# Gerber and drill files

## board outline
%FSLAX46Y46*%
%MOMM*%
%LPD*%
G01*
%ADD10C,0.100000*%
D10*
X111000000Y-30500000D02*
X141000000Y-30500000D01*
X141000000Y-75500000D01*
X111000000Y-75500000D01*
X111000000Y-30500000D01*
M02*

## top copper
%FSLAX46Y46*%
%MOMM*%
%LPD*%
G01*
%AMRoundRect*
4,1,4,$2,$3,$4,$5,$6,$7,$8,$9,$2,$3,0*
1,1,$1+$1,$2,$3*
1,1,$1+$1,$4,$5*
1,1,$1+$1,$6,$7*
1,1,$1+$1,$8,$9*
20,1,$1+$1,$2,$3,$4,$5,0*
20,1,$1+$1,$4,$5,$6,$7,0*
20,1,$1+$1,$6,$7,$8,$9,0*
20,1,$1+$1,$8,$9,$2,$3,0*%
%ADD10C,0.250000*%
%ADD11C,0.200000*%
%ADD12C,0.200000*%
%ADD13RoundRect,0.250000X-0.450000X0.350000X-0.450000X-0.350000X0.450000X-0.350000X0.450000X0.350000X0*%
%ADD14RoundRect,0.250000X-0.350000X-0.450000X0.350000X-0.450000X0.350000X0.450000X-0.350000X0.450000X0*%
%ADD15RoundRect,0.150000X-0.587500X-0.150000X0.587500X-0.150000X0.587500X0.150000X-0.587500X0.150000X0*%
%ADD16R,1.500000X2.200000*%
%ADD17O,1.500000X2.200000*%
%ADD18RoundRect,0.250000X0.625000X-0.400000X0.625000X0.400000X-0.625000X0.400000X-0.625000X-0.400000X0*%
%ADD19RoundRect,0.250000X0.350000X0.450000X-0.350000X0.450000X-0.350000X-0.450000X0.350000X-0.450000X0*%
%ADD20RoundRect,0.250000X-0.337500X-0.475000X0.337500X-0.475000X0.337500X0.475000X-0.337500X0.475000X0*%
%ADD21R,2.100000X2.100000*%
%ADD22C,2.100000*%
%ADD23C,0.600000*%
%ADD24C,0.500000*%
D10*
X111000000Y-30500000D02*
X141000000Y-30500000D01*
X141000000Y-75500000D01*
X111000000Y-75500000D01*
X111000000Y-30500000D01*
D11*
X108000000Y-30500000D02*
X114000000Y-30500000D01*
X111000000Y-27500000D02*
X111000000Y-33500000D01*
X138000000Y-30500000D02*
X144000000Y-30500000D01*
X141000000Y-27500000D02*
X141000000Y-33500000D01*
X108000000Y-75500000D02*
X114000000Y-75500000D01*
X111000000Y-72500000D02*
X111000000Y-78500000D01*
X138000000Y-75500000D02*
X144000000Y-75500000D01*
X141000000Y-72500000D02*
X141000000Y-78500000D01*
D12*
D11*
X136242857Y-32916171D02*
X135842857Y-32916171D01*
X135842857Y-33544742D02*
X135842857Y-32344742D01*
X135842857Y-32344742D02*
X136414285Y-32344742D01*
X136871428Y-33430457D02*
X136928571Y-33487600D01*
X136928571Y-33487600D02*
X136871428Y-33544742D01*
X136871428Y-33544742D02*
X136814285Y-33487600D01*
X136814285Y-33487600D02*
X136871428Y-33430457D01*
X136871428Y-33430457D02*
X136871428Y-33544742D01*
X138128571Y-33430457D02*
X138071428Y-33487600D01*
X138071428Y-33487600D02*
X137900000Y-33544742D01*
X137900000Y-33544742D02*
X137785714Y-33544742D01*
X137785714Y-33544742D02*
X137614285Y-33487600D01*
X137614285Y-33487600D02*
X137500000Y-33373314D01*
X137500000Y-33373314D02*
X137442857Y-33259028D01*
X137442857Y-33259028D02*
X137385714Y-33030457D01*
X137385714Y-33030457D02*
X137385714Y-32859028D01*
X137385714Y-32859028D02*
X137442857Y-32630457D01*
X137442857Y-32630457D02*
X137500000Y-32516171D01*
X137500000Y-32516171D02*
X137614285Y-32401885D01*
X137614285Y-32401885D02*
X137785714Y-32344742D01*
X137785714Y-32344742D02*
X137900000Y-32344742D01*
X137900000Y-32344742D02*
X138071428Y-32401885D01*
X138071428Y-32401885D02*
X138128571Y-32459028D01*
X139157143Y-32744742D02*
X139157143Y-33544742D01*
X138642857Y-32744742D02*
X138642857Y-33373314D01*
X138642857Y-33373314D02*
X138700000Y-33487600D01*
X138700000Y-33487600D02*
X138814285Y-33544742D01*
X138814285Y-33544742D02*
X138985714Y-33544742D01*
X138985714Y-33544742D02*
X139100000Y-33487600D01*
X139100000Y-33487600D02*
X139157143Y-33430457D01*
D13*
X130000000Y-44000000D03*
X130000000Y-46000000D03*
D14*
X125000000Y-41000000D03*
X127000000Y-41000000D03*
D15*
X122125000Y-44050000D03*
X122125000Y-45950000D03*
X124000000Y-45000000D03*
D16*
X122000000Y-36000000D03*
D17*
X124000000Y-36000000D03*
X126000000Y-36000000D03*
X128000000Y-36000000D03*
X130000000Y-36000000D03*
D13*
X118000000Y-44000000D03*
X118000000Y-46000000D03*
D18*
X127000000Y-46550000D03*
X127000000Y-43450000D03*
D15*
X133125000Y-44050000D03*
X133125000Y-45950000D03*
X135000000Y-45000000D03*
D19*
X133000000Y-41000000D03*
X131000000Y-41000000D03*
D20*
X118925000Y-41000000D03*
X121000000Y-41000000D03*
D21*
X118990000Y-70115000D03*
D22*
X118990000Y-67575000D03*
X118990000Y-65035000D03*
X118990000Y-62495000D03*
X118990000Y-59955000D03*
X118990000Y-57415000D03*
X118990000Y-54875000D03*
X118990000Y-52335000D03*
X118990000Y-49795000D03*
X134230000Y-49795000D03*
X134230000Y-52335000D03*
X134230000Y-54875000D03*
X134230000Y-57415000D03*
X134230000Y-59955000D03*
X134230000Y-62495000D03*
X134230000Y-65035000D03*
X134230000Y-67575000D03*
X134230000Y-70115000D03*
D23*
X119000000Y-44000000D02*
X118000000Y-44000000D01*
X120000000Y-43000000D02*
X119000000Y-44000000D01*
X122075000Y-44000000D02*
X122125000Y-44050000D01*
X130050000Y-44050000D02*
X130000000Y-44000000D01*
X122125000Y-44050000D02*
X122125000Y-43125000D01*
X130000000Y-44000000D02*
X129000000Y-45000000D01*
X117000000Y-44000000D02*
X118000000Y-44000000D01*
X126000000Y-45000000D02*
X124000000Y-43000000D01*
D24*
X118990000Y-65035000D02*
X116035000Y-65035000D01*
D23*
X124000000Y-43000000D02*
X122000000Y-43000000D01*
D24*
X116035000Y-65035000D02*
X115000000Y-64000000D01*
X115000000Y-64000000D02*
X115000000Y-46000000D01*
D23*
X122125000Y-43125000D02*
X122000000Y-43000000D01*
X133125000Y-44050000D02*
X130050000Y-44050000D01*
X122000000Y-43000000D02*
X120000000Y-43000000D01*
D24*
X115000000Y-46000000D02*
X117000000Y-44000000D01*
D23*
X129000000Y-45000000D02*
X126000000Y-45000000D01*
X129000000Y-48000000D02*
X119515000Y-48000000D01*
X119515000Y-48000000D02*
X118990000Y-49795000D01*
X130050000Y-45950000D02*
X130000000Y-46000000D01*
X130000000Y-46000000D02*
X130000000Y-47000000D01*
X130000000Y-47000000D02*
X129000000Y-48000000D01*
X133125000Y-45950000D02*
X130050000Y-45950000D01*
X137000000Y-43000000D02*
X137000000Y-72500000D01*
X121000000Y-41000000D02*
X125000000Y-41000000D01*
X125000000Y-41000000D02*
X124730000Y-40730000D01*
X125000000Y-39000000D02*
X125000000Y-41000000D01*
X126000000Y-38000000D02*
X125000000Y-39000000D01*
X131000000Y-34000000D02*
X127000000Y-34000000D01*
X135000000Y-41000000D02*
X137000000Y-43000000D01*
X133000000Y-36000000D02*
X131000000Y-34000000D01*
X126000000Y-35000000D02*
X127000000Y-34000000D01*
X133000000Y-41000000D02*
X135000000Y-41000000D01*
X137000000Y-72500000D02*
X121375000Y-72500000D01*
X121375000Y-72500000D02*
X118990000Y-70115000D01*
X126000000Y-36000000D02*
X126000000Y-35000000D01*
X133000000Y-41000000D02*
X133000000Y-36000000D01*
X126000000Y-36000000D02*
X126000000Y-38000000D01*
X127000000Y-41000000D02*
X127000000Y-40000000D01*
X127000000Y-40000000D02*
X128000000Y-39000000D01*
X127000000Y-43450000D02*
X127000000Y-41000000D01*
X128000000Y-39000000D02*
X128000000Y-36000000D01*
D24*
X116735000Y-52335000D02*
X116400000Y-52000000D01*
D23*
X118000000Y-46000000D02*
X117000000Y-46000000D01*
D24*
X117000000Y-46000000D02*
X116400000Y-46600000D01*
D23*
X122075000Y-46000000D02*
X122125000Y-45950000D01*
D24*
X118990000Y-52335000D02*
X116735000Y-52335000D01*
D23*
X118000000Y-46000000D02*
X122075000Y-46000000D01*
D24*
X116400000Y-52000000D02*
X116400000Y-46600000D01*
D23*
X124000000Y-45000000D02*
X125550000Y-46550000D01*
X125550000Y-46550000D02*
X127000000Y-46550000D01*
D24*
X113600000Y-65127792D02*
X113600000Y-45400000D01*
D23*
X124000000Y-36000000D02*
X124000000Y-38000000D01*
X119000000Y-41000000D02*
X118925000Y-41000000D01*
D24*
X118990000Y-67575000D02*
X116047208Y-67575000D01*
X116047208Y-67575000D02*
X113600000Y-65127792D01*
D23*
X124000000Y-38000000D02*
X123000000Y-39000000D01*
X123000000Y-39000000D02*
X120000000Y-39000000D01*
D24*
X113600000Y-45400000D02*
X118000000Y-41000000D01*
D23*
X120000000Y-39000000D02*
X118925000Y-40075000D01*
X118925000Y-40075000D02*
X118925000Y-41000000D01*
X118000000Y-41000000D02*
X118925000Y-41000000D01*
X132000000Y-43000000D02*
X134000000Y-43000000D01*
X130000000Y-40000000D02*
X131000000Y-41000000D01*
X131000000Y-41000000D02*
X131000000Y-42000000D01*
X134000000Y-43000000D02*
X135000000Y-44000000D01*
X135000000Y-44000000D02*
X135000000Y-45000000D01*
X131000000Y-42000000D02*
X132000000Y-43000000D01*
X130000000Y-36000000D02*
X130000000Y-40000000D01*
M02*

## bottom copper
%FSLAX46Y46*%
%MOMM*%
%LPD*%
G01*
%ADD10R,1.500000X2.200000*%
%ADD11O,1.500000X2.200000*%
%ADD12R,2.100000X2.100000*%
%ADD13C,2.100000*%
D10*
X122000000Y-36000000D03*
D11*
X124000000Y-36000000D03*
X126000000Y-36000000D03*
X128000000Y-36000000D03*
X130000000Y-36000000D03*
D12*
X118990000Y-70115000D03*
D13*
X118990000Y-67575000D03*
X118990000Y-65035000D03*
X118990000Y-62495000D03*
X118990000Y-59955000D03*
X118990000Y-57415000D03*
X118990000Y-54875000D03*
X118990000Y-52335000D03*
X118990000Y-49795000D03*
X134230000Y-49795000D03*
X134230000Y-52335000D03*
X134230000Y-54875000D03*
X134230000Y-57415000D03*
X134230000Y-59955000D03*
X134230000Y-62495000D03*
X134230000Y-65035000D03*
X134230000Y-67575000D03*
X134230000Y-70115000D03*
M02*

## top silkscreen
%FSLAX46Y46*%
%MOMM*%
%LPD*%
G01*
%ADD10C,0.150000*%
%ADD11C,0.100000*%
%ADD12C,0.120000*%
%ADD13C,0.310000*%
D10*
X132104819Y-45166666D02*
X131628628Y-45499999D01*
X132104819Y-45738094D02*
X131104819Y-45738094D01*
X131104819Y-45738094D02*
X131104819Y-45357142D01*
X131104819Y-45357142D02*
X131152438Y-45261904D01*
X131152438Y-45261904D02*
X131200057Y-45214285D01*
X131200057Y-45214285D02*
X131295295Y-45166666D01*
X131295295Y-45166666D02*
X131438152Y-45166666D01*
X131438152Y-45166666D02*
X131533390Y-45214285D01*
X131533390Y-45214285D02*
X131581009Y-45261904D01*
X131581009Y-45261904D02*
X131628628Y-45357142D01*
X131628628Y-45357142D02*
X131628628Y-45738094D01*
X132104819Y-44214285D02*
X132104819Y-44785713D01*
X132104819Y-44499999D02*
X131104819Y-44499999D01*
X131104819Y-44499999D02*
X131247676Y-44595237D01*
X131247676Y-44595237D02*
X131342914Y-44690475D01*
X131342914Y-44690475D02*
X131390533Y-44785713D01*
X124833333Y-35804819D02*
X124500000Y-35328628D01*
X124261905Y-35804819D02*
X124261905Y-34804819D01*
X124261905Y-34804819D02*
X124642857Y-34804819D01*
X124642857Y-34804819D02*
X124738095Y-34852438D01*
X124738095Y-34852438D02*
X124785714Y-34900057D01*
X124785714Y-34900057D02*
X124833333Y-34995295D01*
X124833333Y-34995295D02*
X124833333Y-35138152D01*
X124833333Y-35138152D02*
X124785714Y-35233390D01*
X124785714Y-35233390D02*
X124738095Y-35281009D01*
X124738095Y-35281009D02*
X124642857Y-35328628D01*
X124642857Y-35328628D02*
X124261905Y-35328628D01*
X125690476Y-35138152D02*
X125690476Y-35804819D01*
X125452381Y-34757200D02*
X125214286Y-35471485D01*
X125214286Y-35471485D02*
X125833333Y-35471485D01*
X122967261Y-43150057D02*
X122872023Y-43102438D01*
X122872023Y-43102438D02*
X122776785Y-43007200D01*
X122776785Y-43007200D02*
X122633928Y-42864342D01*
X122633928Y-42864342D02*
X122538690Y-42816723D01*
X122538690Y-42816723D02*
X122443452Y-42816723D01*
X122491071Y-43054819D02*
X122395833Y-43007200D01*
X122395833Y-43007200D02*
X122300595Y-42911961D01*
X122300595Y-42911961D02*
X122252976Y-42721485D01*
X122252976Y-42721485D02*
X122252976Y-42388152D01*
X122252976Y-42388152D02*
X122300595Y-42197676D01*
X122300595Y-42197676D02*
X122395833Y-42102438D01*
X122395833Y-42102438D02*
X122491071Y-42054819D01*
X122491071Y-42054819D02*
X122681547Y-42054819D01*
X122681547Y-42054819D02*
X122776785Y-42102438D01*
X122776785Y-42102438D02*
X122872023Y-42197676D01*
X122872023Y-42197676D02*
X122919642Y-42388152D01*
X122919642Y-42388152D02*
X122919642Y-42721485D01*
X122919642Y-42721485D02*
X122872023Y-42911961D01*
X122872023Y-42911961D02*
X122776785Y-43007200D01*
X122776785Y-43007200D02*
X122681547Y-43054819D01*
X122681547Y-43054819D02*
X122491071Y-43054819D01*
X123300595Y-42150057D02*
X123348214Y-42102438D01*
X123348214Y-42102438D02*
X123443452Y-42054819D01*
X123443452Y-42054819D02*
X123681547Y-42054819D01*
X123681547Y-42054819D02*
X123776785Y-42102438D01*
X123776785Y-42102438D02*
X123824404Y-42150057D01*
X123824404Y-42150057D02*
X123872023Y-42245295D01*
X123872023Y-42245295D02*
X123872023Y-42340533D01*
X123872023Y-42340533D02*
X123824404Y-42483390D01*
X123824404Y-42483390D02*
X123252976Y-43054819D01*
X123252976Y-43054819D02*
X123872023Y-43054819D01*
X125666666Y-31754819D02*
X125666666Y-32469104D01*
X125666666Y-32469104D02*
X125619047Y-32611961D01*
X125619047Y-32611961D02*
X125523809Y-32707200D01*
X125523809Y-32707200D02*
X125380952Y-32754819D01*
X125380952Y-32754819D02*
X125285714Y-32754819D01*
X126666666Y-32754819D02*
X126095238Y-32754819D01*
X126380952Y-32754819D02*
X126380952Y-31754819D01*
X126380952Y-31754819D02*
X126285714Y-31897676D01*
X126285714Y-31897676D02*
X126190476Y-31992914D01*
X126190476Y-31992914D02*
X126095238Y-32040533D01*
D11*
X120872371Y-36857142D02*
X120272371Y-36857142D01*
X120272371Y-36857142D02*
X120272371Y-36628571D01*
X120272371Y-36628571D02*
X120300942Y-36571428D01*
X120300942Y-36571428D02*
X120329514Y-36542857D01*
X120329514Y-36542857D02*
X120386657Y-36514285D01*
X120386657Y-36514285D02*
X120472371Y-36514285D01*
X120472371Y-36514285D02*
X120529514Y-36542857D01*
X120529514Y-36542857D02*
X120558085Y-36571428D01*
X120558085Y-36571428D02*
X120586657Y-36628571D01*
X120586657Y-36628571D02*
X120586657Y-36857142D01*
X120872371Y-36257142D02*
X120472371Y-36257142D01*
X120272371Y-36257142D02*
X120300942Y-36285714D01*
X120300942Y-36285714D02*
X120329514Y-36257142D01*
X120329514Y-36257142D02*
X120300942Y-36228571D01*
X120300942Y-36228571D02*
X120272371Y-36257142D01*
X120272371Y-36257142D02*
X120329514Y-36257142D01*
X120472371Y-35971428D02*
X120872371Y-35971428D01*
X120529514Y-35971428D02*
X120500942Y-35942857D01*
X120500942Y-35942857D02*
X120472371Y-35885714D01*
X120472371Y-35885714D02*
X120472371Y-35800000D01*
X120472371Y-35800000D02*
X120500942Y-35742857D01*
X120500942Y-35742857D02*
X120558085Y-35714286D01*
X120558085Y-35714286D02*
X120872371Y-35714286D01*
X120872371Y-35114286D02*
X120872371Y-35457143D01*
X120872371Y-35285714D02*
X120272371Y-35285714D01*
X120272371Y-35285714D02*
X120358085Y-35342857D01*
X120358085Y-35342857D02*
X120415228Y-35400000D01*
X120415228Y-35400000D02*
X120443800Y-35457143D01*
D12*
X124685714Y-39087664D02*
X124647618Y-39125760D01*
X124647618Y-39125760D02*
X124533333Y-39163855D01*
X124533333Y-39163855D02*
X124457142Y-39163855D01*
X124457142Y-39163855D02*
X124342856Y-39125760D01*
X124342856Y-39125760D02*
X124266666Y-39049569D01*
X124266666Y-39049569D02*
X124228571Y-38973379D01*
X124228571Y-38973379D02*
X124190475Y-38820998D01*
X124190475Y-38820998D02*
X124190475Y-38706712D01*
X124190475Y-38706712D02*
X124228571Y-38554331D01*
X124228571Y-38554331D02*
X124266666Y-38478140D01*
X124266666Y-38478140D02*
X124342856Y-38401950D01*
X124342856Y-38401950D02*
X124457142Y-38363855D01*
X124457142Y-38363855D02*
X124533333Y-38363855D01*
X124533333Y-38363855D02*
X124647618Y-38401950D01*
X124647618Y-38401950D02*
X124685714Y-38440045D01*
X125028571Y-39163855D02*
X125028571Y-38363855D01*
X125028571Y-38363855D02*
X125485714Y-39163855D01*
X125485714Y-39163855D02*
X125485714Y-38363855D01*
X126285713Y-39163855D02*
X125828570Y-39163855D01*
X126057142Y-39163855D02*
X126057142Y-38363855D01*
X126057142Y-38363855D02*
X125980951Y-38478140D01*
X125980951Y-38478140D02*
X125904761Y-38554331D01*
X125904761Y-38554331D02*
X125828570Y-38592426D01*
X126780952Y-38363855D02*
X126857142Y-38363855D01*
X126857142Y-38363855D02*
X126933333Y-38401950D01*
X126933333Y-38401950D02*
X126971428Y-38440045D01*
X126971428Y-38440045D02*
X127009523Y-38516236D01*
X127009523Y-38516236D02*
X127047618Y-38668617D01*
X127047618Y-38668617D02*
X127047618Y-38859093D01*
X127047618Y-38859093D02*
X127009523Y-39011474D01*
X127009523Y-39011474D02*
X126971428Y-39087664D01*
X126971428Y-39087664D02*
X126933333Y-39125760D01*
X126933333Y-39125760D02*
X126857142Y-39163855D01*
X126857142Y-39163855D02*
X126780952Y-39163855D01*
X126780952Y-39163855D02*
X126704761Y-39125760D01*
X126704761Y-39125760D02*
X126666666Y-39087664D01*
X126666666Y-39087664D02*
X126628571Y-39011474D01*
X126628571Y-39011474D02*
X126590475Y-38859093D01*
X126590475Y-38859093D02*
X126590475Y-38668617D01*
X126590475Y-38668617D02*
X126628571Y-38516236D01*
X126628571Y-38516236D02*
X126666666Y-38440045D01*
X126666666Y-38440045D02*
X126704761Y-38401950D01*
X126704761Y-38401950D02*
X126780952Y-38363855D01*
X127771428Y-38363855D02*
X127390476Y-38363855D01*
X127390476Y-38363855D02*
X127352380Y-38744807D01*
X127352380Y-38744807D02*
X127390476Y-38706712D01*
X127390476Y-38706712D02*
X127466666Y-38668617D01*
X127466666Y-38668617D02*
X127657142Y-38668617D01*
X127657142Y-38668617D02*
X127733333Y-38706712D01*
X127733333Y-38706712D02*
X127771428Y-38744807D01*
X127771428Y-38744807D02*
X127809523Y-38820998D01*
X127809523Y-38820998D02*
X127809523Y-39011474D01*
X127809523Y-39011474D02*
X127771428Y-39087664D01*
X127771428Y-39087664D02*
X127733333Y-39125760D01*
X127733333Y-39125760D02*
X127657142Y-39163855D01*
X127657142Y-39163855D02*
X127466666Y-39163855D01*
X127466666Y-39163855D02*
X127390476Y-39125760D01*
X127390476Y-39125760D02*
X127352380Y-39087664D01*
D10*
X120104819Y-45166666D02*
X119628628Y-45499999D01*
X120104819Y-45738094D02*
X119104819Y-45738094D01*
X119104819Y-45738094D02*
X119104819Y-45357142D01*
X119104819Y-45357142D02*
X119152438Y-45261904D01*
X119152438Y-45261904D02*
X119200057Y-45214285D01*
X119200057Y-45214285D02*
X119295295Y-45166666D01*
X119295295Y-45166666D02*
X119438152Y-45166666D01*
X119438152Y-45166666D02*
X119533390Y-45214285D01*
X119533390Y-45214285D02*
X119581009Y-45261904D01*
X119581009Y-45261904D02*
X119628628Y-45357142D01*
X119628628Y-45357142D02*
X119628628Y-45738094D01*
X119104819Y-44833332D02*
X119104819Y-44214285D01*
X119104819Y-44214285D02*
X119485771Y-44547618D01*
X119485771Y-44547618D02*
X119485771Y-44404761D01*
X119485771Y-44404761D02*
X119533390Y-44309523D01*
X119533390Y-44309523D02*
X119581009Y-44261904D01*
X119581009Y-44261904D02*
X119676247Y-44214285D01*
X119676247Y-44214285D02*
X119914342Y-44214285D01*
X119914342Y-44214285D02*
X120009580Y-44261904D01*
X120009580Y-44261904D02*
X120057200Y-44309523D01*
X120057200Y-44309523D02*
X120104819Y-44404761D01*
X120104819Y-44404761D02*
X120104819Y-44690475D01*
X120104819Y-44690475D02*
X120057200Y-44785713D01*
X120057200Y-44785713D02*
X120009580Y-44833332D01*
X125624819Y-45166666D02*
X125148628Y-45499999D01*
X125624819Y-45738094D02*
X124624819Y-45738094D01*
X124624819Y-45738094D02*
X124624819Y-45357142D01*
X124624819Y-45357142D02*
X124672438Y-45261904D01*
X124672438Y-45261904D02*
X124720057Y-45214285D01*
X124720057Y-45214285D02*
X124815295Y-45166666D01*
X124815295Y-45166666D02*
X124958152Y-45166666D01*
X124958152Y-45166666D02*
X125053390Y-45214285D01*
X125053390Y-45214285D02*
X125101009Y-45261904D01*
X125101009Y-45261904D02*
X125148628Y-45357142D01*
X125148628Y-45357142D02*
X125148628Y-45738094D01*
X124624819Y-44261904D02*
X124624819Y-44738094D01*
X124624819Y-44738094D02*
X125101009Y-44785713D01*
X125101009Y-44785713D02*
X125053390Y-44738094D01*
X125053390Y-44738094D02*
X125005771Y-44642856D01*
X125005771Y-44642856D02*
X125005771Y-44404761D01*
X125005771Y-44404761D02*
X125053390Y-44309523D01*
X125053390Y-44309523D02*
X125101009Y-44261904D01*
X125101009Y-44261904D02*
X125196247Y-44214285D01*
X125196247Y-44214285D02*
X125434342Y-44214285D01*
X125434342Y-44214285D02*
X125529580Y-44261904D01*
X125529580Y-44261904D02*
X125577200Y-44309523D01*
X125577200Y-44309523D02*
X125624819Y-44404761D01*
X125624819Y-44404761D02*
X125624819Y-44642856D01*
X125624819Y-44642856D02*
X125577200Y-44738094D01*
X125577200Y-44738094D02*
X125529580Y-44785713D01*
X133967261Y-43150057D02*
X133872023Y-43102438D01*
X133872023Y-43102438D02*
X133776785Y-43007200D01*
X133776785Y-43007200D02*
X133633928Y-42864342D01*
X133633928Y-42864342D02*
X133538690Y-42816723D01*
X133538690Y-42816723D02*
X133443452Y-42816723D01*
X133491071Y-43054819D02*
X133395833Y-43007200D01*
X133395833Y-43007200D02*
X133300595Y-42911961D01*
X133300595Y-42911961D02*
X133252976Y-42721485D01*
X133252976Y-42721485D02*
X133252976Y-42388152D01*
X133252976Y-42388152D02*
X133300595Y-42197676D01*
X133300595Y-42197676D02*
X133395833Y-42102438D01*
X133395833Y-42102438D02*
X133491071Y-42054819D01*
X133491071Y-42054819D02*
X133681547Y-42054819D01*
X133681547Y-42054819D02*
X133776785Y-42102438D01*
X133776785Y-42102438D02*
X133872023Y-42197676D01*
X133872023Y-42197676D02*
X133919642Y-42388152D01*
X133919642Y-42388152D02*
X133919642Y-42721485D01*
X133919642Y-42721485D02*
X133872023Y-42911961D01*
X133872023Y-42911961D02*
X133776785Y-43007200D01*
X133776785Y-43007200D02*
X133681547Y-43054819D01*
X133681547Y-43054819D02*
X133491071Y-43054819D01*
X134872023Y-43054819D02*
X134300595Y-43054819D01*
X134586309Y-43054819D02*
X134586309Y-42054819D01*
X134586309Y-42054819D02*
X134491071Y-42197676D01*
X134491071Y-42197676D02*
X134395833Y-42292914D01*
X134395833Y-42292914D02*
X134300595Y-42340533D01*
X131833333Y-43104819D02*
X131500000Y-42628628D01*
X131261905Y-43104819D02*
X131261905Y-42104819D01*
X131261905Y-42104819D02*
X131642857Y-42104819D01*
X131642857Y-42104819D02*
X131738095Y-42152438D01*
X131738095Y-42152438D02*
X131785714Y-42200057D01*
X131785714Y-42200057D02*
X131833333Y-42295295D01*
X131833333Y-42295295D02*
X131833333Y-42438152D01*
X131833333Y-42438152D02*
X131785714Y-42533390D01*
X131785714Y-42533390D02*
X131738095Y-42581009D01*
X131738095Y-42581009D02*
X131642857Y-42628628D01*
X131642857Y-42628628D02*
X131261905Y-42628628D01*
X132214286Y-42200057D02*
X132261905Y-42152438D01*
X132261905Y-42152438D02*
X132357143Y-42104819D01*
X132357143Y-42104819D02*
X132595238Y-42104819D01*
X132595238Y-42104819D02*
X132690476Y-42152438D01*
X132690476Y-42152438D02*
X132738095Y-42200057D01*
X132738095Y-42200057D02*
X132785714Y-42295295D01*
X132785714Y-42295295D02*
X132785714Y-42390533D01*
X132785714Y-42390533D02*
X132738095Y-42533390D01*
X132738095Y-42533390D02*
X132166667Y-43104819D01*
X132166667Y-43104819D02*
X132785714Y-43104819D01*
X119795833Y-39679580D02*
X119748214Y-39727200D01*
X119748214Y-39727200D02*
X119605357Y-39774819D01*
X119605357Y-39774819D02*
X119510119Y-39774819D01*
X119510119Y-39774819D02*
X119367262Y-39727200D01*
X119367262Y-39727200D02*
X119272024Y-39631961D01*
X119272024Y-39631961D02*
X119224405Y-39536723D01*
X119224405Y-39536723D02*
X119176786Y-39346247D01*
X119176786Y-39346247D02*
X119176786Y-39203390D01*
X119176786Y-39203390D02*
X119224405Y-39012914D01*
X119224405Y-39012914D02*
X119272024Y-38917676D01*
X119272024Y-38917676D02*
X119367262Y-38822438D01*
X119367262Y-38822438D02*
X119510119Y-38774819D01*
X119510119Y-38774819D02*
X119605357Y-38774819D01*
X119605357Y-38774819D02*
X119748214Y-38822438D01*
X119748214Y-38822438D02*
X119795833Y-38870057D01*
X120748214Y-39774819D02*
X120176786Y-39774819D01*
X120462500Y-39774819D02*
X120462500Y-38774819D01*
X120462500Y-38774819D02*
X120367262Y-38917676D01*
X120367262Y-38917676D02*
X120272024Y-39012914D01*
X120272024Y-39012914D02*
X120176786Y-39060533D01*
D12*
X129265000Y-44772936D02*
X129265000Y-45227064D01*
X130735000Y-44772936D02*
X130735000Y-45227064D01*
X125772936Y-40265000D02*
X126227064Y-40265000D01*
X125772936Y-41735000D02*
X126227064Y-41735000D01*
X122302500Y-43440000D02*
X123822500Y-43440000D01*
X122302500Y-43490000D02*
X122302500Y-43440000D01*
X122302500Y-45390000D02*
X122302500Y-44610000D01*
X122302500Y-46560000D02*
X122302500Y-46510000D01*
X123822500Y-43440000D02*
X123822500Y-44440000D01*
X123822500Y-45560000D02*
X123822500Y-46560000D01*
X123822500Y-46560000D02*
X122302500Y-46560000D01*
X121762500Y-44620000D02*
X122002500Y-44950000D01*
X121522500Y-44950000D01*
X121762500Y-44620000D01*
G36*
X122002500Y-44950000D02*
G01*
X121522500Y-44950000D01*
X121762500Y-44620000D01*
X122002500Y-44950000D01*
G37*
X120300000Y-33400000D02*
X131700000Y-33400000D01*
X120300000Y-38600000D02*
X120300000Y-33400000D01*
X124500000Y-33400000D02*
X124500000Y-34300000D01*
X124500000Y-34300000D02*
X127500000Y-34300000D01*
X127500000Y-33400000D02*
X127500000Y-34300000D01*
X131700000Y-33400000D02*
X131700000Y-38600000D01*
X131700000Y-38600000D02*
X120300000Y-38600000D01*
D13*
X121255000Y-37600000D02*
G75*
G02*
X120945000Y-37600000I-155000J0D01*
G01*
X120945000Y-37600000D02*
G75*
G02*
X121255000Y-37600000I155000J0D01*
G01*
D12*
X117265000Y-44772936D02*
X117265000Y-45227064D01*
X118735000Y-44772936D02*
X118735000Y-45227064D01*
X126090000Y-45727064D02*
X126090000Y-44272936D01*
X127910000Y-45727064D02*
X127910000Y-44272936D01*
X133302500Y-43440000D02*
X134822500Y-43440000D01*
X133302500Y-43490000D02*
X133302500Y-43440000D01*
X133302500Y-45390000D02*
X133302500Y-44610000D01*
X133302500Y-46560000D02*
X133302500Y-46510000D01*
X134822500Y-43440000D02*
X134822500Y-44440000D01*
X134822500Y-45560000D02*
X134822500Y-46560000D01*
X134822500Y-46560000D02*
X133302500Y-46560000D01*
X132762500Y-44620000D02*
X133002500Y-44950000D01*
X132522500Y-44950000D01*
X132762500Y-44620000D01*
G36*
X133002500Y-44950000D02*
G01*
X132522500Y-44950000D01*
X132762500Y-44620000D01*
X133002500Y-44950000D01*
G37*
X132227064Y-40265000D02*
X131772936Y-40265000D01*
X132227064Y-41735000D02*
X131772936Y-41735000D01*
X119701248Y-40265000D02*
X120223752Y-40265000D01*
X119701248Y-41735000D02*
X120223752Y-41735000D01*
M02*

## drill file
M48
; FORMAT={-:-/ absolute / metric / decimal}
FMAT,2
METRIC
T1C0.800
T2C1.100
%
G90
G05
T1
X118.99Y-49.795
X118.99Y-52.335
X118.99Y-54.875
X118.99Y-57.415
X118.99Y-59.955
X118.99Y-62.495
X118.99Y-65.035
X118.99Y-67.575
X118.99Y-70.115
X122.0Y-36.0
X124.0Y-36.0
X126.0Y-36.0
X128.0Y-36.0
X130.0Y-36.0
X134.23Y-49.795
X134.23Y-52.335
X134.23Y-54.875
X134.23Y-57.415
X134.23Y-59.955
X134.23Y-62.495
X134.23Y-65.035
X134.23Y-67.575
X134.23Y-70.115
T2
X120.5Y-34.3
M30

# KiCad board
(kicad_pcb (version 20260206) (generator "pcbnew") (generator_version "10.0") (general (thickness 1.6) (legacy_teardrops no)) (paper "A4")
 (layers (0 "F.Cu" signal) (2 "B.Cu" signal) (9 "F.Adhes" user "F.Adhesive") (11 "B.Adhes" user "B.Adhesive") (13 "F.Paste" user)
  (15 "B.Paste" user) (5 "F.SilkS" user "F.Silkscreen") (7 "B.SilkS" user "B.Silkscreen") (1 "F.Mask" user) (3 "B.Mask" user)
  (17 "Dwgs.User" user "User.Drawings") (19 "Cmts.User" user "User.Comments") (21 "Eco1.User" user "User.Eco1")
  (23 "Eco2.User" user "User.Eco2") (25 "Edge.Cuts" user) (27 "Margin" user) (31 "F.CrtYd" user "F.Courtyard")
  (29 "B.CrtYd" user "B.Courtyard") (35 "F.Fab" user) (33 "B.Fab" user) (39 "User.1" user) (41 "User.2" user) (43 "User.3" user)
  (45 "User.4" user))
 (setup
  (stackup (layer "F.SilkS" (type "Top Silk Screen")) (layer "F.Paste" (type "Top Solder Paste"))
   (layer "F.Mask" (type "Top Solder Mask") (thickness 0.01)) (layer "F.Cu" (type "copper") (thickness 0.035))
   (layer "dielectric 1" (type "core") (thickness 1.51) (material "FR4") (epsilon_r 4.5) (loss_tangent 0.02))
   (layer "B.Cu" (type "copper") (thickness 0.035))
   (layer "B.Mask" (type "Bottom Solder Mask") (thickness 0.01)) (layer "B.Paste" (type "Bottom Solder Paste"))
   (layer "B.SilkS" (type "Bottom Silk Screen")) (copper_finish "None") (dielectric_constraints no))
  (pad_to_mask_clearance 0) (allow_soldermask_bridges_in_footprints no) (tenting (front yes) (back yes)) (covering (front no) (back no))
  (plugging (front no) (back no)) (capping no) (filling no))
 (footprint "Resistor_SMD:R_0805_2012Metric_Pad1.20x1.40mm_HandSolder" (layer "F.Cu") (at 130 45 -90)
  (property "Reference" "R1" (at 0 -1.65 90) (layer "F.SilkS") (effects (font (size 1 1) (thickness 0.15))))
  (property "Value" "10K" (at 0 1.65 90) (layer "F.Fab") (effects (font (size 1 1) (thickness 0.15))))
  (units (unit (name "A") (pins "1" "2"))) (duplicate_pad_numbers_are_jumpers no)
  (fp_line (start -0.227064 0.735) (end 0.227064 0.735) (stroke (width 0.12) (type solid)) (layer "F.SilkS"))
  (fp_line (start -0.227064 -0.735) (end 0.227064 -0.735) (stroke (width 0.12) (type solid)) (layer "F.SilkS"))
  (pad "1" smd roundrect (at -1 0 270) (size 1.2 1.4) (layers "F.Cu" "F.Mask" "F.Paste") (roundrect_rratio 0.208333) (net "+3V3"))
  (pad "2" smd roundrect (at 1 0 270) (size 1.2 1.4) (layers "F.Cu" "F.Mask" "F.Paste") (roundrect_rratio 0.208333) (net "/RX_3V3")))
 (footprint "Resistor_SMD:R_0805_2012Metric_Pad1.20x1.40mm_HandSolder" (layer "F.Cu") (at 126 41)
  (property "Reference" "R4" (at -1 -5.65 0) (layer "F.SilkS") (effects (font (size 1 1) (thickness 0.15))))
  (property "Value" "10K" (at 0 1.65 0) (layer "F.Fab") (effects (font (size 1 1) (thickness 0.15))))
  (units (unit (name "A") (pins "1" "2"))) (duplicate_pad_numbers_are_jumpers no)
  (fp_line (start -0.227064 -0.735) (end 0.227064 -0.735) (stroke (width 0.12) (type solid)) (layer "F.SilkS"))
  (fp_line (start -0.227064 0.735) (end 0.227064 0.735) (stroke (width 0.12) (type solid)) (layer "F.SilkS"))
  (pad "1" smd roundrect (at -1 0) (size 1.2 1.4) (layers "F.Cu" "F.Mask" "F.Paste") (roundrect_rratio 0.208333) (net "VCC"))
  (pad "2" smd roundrect (at 1 0) (size 1.2 1.4) (layers "F.Cu" "F.Mask" "F.Paste") (roundrect_rratio 0.208333) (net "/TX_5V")))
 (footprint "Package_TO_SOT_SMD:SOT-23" (layer "F.Cu") (at 123.0625 45)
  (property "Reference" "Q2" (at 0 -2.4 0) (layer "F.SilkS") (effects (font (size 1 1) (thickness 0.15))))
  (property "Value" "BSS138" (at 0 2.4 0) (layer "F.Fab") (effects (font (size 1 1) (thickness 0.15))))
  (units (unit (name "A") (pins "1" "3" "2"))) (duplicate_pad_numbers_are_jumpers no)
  (fp_line (start -0.76 -1.56) (end 0.76 -1.56) (stroke (width 0.12) (type solid)) (layer "F.SilkS"))
  (fp_line (start -0.76 -1.51) (end -0.76 -1.56) (stroke (width 0.12) (type solid)) (layer "F.SilkS"))
  (fp_line (start -0.76 0.39) (end -0.76 -0.39) (stroke (width 0.12) (type solid)) (layer "F.SilkS"))
  (fp_line (start -0.76 1.56) (end -0.76 1.51) (stroke (width 0.12) (type solid)) (layer "F.SilkS"))
  (fp_line (start 0.76 -1.56) (end 0.76 -0.56) (stroke (width 0.12) (type solid)) (layer "F.SilkS"))
  (fp_line (start 0.76 0.56) (end 0.76 1.56) (stroke (width 0.12) (type solid)) (layer "F.SilkS"))
  (fp_line (start 0.76 1.56) (end -0.76 1.56) (stroke (width 0.12) (type solid)) (layer "F.SilkS"))
  (fp_poly (pts (xy -1.3 -0.38) (xy -1.06 -0.05) (xy -1.54 -0.05)) (stroke (width 0.12) (type solid)) (fill yes) (layer "F.SilkS"))
  (pad "1" smd roundrect (at -0.9375 -0.95) (size 1.475 0.6) (layers "F.Cu" "F.Mask" "F.Paste") (roundrect_rratio 0.25) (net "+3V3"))
  (pad "2" smd roundrect (at -0.9375 0.95) (size 1.475 0.6) (layers "F.Cu" "F.Mask" "F.Paste") (roundrect_rratio 0.25) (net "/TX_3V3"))
  (pad "3" smd roundrect (at 0.9375 0) (size 1.475 0.6) (layers "F.Cu" "F.Mask" "F.Paste") (roundrect_rratio 0.25) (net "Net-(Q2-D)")))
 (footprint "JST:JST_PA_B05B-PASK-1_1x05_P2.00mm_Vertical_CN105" (layer "F.Cu") (at 122 36)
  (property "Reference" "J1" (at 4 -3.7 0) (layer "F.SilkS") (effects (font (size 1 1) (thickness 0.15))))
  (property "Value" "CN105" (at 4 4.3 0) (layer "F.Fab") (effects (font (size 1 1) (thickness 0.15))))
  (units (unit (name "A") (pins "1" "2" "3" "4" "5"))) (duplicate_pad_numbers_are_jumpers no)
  (fp_line (start -1.7 -2.6) (end 9.7 -2.6) (stroke (width 0.12) (type solid)) (layer "F.SilkS"))
  (fp_line (start -1.7 2.6) (end -1.7 -2.6) (stroke (width 0.12) (type solid)) (layer "F.SilkS"))
  (fp_line (start 2.5 -2.6) (end 2.5 -1.7) (stroke (width 0.12) (type solid)) (layer "F.SilkS"))
  (fp_line (start 2.5 -1.7) (end 5.5 -1.7) (stroke (width 0.12) (type solid)) (layer "F.SilkS"))
  (fp_line (start 5.5 -2.6) (end 5.5 -1.7) (stroke (width 0.12) (type solid)) (layer "F.SilkS"))
  (fp_line (start 9.7 -2.6) (end 9.7 2.6) (stroke (width 0.12) (type solid)) (layer "F.SilkS"))
  (fp_line (start 9.7 2.6) (end -1.7 2.6) (stroke (width 0.12) (type solid)) (layer "F.SilkS"))
  (fp_circle (center -0.9 1.6) (end -0.65 1.6) (stroke (width 0.12) (type solid)) (fill yes) (layer "F.SilkS"))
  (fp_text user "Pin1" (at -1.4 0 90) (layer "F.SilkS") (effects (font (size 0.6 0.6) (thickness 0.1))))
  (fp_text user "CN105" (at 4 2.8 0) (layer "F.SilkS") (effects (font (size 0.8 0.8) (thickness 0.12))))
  (pad "" np_thru_hole circle (at -1.5 -1.7) (size 1.1 1.1) (drill 1.1) (layers "*.Cu" "*.Mask"))
  (pad "1" thru_hole rect (at 0 0) (size 1.5 2.2) (drill 0.8) (layers "*.Cu" "*.Mask") (remove_unused_layers no)
   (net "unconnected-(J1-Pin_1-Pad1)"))
  (pad "2" thru_hole oval (at 2 0) (size 1.5 2.2) (drill 0.8) (layers "*.Cu" "*.Mask") (remove_unused_layers no) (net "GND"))
  (pad "3" thru_hole oval (at 4 0) (size 1.5 2.2) (drill 0.8) (layers "*.Cu" "*.Mask") (remove_unused_layers no) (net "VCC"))
  (pad "4" thru_hole oval (at 6 0) (size 1.5 2.2) (drill 0.8) (layers "*.Cu" "*.Mask") (remove_unused_layers no) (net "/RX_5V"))
  (pad "5" thru_hole oval (at 8 0) (size 1.5 2.2) (drill 0.8) (layers "*.Cu" "*.Mask") (remove_unused_layers no) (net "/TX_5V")))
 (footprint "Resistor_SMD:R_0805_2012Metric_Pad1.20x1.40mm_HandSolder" (layer "F.Cu") (at 118 45 -90)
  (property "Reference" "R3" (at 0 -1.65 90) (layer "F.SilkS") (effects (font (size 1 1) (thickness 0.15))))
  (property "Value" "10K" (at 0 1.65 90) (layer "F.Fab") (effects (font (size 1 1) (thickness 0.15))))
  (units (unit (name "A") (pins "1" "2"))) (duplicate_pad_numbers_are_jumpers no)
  (fp_line (start -0.227064 0.735) (end 0.227064 0.735) (stroke (width 0.12) (type solid)) (layer "F.SilkS"))
  (fp_line (start -0.227064 -0.735) (end 0.227064 -0.735) (stroke (width 0.12) (type solid)) (layer "F.SilkS"))
  (pad "1" smd roundrect (at -1 0 270) (size 1.2 1.4) (layers "F.Cu" "F.Mask" "F.Paste") (roundrect_rratio 0.208333) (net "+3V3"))
  (pad "2" smd roundrect (at 1 0 270) (size 1.2 1.4) (layers "F.Cu" "F.Mask" "F.Paste") (roundrect_rratio 0.208333) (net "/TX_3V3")))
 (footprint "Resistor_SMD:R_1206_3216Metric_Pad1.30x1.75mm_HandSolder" (layer "F.Cu") (at 127 45 90)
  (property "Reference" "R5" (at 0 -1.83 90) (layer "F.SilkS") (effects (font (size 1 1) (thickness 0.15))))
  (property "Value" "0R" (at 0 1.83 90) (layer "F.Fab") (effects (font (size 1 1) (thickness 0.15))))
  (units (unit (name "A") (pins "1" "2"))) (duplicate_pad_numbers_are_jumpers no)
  (fp_line (start -0.727064 -0.91) (end 0.727064 -0.91) (stroke (width 0.12) (type solid)) (layer "F.SilkS"))
  (fp_line (start -0.727064 0.91) (end 0.727064 0.91) (stroke (width 0.12) (type solid)) (layer "F.SilkS"))
  (pad "1" smd roundrect (at -1.55 0 90) (size 1.3 1.75) (layers "F.Cu" "F.Mask" "F.Paste") (roundrect_rratio 0.192308) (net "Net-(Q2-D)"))
  (pad "2" smd roundrect (at 1.55 0 90) (size 1.3 1.75) (layers "F.Cu" "F.Mask" "F.Paste") (roundrect_rratio 0.192308) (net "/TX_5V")))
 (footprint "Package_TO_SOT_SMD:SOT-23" (layer "F.Cu") (at 134.0625 45)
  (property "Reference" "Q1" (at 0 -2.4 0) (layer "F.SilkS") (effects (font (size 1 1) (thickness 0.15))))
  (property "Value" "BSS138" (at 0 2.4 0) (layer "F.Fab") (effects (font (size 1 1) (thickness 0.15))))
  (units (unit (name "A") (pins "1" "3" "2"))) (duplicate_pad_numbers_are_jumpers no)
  (fp_line (start -0.76 -1.56) (end 0.76 -1.56) (stroke (width 0.12) (type solid)) (layer "F.SilkS"))
  (fp_line (start -0.76 -1.51) (end -0.76 -1.56) (stroke (width 0.12) (type solid)) (layer "F.SilkS"))
  (fp_line (start -0.76 0.39) (end -0.76 -0.39) (stroke (width 0.12) (type solid)) (layer "F.SilkS"))
  (fp_line (start -0.76 1.56) (end -0.76 1.51) (stroke (width 0.12) (type solid)) (layer "F.SilkS"))
  (fp_line (start 0.76 -1.56) (end 0.76 -0.56) (stroke (width 0.12) (type solid)) (layer "F.SilkS"))
  (fp_line (start 0.76 0.56) (end 0.76 1.56) (stroke (width 0.12) (type solid)) (layer "F.SilkS"))
  (fp_line (start 0.76 1.56) (end -0.76 1.56) (stroke (width 0.12) (type solid)) (layer "F.SilkS"))
  (fp_poly (pts (xy -1.3 -0.38) (xy -1.06 -0.05) (xy -1.54 -0.05)) (stroke (width 0.12) (type solid)) (fill yes) (layer "F.SilkS"))
  (pad "1" smd roundrect (at -0.9375 -0.95) (size 1.475 0.6) (layers "F.Cu" "F.Mask" "F.Paste") (roundrect_rratio 0.25) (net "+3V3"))
  (pad "2" smd roundrect (at -0.9375 0.95) (size 1.475 0.6) (layers "F.Cu" "F.Mask" "F.Paste") (roundrect_rratio 0.25) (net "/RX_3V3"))
  (pad "3" smd roundrect (at 0.9375 0) (size 1.475 0.6) (layers "F.Cu" "F.Mask" "F.Paste") (roundrect_rratio 0.25) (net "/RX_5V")))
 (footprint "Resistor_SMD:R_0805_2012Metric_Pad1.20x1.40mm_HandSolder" (layer "F.Cu") (at 132 41 180)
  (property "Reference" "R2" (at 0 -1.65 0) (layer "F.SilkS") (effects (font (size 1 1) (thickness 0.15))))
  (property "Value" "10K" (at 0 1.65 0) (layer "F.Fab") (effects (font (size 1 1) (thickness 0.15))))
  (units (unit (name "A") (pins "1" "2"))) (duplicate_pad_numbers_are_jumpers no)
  (fp_line (start -0.227064 0.735) (end 0.227064 0.735) (stroke (width 0.12) (type solid)) (layer "F.SilkS"))
  (fp_line (start -0.227064 -0.735) (end 0.227064 -0.735) (stroke (width 0.12) (type solid)) (layer "F.SilkS"))
  (pad "1" smd roundrect (at -1 0 180) (size 1.2 1.4) (layers "F.Cu" "F.Mask" "F.Paste") (roundrect_rratio 0.208333) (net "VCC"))
  (pad "2" smd roundrect (at 1 0 180) (size 1.2 1.4) (layers "F.Cu" "F.Mask" "F.Paste") (roundrect_rratio 0.208333) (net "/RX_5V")))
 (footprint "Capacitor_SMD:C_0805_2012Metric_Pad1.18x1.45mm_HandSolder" (layer "F.Cu") (at 119.9625 41)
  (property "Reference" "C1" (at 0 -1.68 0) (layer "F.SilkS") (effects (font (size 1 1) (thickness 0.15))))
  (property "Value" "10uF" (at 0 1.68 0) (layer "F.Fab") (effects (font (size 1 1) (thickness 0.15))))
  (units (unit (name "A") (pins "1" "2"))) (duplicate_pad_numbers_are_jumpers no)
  (fp_line (start -0.261252 -0.735) (end 0.261252 -0.735) (stroke (width 0.12) (type solid)) (layer "F.SilkS"))
  (fp_line (start -0.261252 0.735) (end 0.261252 0.735) (stroke (width 0.12) (type solid)) (layer "F.SilkS"))
  (pad "1" smd roundrect (at -1.0375 0) (size 1.175 1.45) (layers "F.Cu" "F.Mask" "F.Paste") (roundrect_rratio 0.212766) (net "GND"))
  (pad "2" smd roundrect (at 1.0375 0) (size 1.175 1.45) (layers "F.Cu" "F.Mask" "F.Paste") (roundrect_rratio 0.212766) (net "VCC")))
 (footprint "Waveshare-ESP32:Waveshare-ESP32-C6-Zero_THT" (layer "B.Cu") (at 126.61 70.115)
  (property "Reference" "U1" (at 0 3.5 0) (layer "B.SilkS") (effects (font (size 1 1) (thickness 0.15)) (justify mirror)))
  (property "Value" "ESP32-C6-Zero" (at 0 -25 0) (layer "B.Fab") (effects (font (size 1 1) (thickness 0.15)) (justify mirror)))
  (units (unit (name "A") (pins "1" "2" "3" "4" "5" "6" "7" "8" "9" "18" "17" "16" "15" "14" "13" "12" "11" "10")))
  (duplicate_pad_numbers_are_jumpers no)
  (pad "1" thru_hole rect (at -7.62 0) (size 2.1 2.1) (drill 0.8) (layers "*.Cu" "*.Mask") (remove_unused_layers no) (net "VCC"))
  (pad "2" thru_hole circle (at -7.62 -2.54) (size 2.1 2.1) (drill 0.8) (layers "*.Cu" "*.Mask") (remove_unused_layers no) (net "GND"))
  (pad "3" thru_hole circle (at -7.62 -5.08) (size 2.1 2.1) (drill 0.8) (layers "*.Cu" "*.Mask") (remove_unused_layers no) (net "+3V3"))
  (pad "4" thru_hole circle (at -7.62 -7.62) (size 2.1 2.1) (drill 0.8) (layers "*.Cu" "*.Mask") (remove_unused_layers no)
   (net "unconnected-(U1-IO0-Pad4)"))
  (pad "5" thru_hole circle (at -7.62 -10.16) (size 2.1 2.1) (drill 0.8) (layers "*.Cu" "*.Mask") (remove_unused_layers no)
   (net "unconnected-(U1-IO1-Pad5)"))
  (pad "6" thru_hole circle (at -7.62 -12.7) (size 2.1 2.1) (drill 0.8) (layers "*.Cu" "*.Mask") (remove_unused_layers no)
   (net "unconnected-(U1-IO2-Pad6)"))
  (pad "7" thru_hole circle (at -7.62 -15.24) (size 2.1 2.1) (drill 0.8) (layers "*.Cu" "*.Mask") (remove_unused_layers no)
   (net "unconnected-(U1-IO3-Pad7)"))
  (pad "8" thru_hole circle (at -7.62 -17.78) (size 2.1 2.1) (drill 0.8) (layers "*.Cu" "*.Mask") (remove_unused_layers no) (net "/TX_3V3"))
  (pad "9" thru_hole circle (at -7.62 -20.32) (size 2.1 2.1) (drill 0.8) (layers "*.Cu" "*.Mask") (remove_unused_layers no) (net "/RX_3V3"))
  (pad "10" thru_hole circle (at 7.62 -20.32) (size 2.1 2.1) (drill 0.8) (layers "*.Cu" "*.Mask") (remove_unused_layers no)
   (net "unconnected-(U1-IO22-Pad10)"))
  (pad "11" thru_hole circle (at 7.62 -17.78) (size 2.1 2.1) (drill 0.8) (layers "*.Cu" "*.Mask") (remove_unused_layers no)
   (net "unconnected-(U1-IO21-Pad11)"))
  (pad "12" thru_hole circle (at 7.62 -15.24) (size 2.1 2.1) (drill 0.8) (layers "*.Cu" "*.Mask") (remove_unused_layers no)
   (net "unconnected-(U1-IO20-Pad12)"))
  (pad "13" thru_hole circle (at 7.62 -12.7) (size 2.1 2.1) (drill 0.8) (layers "*.Cu" "*.Mask") (remove_unused_layers no)
   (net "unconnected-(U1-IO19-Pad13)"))
  (pad "14" thru_hole circle (at 7.62 -10.16) (size 2.1 2.1) (drill 0.8) (layers "*.Cu" "*.Mask") (remove_unused_layers no)
   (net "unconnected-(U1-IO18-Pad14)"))
  (pad "15" thru_hole circle (at 7.62 -7.62) (size 2.1 2.1) (drill 0.8) (layers "*.Cu" "*.Mask") (remove_unused_layers no)
   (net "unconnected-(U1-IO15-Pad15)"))
  (pad "16" thru_hole circle (at 7.62 -5.08) (size 2.1 2.1) (drill 0.8) (layers "*.Cu" "*.Mask") (remove_unused_layers no)
   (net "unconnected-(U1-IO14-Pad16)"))
  (pad "17" thru_hole circle (at 7.62 -2.54) (size 2.1 2.1) (drill 0.8) (layers "*.Cu" "*.Mask") (remove_unused_layers no)
   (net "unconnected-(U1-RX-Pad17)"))
  (pad "18" thru_hole circle (at 7.62 0) (size 2.1 2.1) (drill 0.8) (layers "*.Cu" "*.Mask") (remove_unused_layers no)
   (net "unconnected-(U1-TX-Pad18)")))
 (gr_rect (start 111 30.5) (end 141 75.5) (stroke (width 0.1) (type default)) (fill no) (layer "Edge.Cuts"))
 (gr_rect (start 111 30.5) (end 141 75.5) (stroke (width 0.25) (type default)) (fill no) (layer "F.Cu"))
 (gr_line (start 108 30.5) (end 114 30.5) (stroke (width 0.2) (type default)) (layer "F.Cu"))
 (gr_line (start 111 27.5) (end 111 33.5) (stroke (width 0.2) (type default)) (layer "F.Cu"))
 (gr_line (start 138 30.5) (end 144 30.5) (stroke (width 0.2) (type default)) (layer "F.Cu"))
 (gr_line (start 141 27.5) (end 141 33.5) (stroke (width 0.2) (type default)) (layer "F.Cu"))
 (gr_line (start 108 75.5) (end 114 75.5) (stroke (width 0.2) (type default)) (layer "F.Cu"))
 (gr_line (start 111 72.5) (end 111 78.5) (stroke (width 0.2) (type default)) (layer "F.Cu"))
 (gr_line (start 138 75.5) (end 144 75.5) (stroke (width 0.2) (type default)) (layer "F.Cu"))
 (gr_line (start 141 72.5) (end 141 78.5) (stroke (width 0.2) (type default)) (layer "F.Cu"))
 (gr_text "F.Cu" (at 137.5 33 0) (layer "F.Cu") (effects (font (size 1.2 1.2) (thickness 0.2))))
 (segment (start 119 44) (end 118 44) (width 0.6) (layer "F.Cu") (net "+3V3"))
 (segment (start 120 43) (end 119 44) (width 0.6) (layer "F.Cu") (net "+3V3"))
 (segment (start 122.075 44) (end 122.125 44.05) (width 0.6) (layer "F.Cu") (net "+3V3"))
 (segment (start 130.05 44.05) (end 130 44) (width 0.6) (layer "F.Cu") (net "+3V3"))
 (segment (start 122.125 44.05) (end 122.125 43.125) (width 0.6) (layer "F.Cu") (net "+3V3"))
 (segment (start 130 44) (end 129 45) (width 0.6) (layer "F.Cu") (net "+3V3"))
 (segment (start 117 44) (end 118 44) (width 0.6) (layer "F.Cu") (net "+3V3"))
 (segment (start 126 45) (end 124 43) (width 0.6) (layer "F.Cu") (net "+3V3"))
 (segment (start 118.99 65.035) (end 116.035 65.035) (width 0.5) (layer "F.Cu") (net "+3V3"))
 (segment (start 124 43) (end 122 43) (width 0.6) (layer "F.Cu") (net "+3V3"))
 (segment (start 116.035 65.035) (end 115 64) (width 0.5) (layer "F.Cu") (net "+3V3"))
 (segment (start 115 64) (end 115 46) (width 0.5) (layer "F.Cu") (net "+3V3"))
 (segment (start 122.125 43.125) (end 122 43) (width 0.6) (layer "F.Cu") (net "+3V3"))
 (segment (start 133.125 44.05) (end 130.05 44.05) (width 0.6) (layer "F.Cu") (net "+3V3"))
 (segment (start 122 43) (end 120 43) (width 0.6) (layer "F.Cu") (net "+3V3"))
 (segment (start 115 46) (end 117 44) (width 0.5) (layer "F.Cu") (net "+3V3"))
 (segment (start 129 45) (end 126 45) (width 0.6) (layer "F.Cu") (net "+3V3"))
 (segment (start 129 48) (end 119.515 48) (width 0.6) (layer "F.Cu") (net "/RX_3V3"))
 (segment (start 119.515 48) (end 118.99 49.795) (width 0.6) (layer "F.Cu") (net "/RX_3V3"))
 (segment (start 130.05 45.95) (end 130 46) (width 0.6) (layer "F.Cu") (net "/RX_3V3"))
 (segment (start 130 46) (end 130 47) (width 0.6) (layer "F.Cu") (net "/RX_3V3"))
 (segment (start 130 47) (end 129 48) (width 0.6) (layer "F.Cu") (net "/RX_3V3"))
 (segment (start 133.125 45.95) (end 130.05 45.95) (width 0.6) (layer "F.Cu") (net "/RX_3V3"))
 (segment (start 137 43) (end 137 72.5) (width 0.6) (layer "F.Cu") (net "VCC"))
 (segment (start 121 41) (end 125 41) (width 0.6) (layer "F.Cu") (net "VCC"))
 (segment (start 125 41) (end 124.73 40.73) (width 0.6) (layer "F.Cu") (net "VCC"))
 (segment (start 125 39) (end 125 41) (width 0.6) (layer "F.Cu") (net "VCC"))
 (segment (start 126 38) (end 125 39) (width 0.6) (layer "F.Cu") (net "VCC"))
 (segment (start 131 34) (end 127 34) (width 0.6) (layer "F.Cu") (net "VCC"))
 (segment (start 135 41) (end 137 43) (width 0.6) (layer "F.Cu") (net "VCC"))
 (segment (start 133 36) (end 131 34) (width 0.6) (layer "F.Cu") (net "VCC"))
 (segment (start 126 35) (end 127 34) (width 0.6) (layer "F.Cu") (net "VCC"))
 (segment (start 133 41) (end 135 41) (width 0.6) (layer "F.Cu") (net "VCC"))
 (segment (start 137 72.5) (end 121.375 72.5) (width 0.6) (layer "F.Cu") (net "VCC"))
 (segment (start 121.375 72.5) (end 118.99 70.115) (width 0.6) (layer "F.Cu") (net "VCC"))
 (segment (start 126 36) (end 126 35) (width 0.6) (layer "F.Cu") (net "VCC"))
 (segment (start 133 41) (end 133 36) (width 0.6) (layer "F.Cu") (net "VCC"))
 (segment (start 126 36) (end 126 38) (width 0.6) (layer "F.Cu") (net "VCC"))
 (segment (start 127 41) (end 127 40) (width 0.6) (layer "F.Cu") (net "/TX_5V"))
 (segment (start 127 40) (end 128 39) (width 0.6) (layer "F.Cu") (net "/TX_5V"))
 (segment (start 127 43.45) (end 127 41) (width 0.6) (layer "F.Cu") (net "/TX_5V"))
 (segment (start 128 39) (end 128 36) (width 0.6) (layer "F.Cu") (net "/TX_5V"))
 (segment (start 116.735 52.335) (end 116.4 52) (width 0.5) (layer "F.Cu") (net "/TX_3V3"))
 (segment (start 118 46) (end 117 46) (width 0.6) (layer "F.Cu") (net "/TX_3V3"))
 (segment (start 117 46) (end 116.4 46.6) (width 0.5) (layer "F.Cu") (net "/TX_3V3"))
 (segment (start 122.075 46) (end 122.125 45.95) (width 0.6) (layer "F.Cu") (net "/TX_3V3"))
 (segment (start 118.99 52.335) (end 116.735 52.335) (width 0.5) (layer "F.Cu") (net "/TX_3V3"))
 (segment (start 118 46) (end 122.075 46) (width 0.6) (layer "F.Cu") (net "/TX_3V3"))
 (segment (start 116.4 52) (end 116.4 46.6) (width 0.5) (layer "F.Cu") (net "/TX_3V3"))
 (segment (start 124 45) (end 125.55 46.55) (width 0.6) (layer "F.Cu") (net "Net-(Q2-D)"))
 (segment (start 125.55 46.55) (end 127 46.55) (width 0.6) (layer "F.Cu") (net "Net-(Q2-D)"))
 (segment (start 113.6 65.127792) (end 113.6 45.4) (width 0.5) (layer "F.Cu") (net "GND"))
 (segment (start 124 36) (end 124 38) (width 0.6) (layer "F.Cu") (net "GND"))
 (segment (start 119 41) (end 118.925 41) (width 0.6) (layer "F.Cu") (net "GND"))
 (segment (start 118.99 67.575) (end 116.047208 67.575) (width 0.5) (layer "F.Cu") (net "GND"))
 (segment (start 116.047208 67.575) (end 113.6 65.127792) (width 0.5) (layer "F.Cu") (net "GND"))
 (segment (start 124 38) (end 123 39) (width 0.6) (layer "F.Cu") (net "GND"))
 (segment (start 123 39) (end 120 39) (width 0.6) (layer "F.Cu") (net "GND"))
 (segment (start 113.6 45.4) (end 118 41) (width 0.5) (layer "F.Cu") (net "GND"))
 (segment (start 120 39) (end 118.925 40.075) (width 0.6) (layer "F.Cu") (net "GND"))
 (segment (start 118.925 40.075) (end 118.925 41) (width 0.6) (layer "F.Cu") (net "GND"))
 (segment (start 118 41) (end 118.925 41) (width 0.6) (layer "F.Cu") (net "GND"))
 (segment (start 132 43) (end 134 43) (width 0.6) (layer "F.Cu") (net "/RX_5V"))
 (segment (start 130 40) (end 131 41) (width 0.6) (layer "F.Cu") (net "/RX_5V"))
 (segment (start 131 41) (end 131 42) (width 0.6) (layer "F.Cu") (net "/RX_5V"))
 (segment (start 134 43) (end 135 44) (width 0.6) (layer "F.Cu") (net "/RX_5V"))
 (segment (start 135 44) (end 135 45) (width 0.6) (layer "F.Cu") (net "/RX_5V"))
 (segment (start 131 42) (end 132 43) (width 0.6) (layer "F.Cu") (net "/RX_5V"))
 (segment (start 130 36) (end 130 40) (width 0.6) (layer "F.Cu") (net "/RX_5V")))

